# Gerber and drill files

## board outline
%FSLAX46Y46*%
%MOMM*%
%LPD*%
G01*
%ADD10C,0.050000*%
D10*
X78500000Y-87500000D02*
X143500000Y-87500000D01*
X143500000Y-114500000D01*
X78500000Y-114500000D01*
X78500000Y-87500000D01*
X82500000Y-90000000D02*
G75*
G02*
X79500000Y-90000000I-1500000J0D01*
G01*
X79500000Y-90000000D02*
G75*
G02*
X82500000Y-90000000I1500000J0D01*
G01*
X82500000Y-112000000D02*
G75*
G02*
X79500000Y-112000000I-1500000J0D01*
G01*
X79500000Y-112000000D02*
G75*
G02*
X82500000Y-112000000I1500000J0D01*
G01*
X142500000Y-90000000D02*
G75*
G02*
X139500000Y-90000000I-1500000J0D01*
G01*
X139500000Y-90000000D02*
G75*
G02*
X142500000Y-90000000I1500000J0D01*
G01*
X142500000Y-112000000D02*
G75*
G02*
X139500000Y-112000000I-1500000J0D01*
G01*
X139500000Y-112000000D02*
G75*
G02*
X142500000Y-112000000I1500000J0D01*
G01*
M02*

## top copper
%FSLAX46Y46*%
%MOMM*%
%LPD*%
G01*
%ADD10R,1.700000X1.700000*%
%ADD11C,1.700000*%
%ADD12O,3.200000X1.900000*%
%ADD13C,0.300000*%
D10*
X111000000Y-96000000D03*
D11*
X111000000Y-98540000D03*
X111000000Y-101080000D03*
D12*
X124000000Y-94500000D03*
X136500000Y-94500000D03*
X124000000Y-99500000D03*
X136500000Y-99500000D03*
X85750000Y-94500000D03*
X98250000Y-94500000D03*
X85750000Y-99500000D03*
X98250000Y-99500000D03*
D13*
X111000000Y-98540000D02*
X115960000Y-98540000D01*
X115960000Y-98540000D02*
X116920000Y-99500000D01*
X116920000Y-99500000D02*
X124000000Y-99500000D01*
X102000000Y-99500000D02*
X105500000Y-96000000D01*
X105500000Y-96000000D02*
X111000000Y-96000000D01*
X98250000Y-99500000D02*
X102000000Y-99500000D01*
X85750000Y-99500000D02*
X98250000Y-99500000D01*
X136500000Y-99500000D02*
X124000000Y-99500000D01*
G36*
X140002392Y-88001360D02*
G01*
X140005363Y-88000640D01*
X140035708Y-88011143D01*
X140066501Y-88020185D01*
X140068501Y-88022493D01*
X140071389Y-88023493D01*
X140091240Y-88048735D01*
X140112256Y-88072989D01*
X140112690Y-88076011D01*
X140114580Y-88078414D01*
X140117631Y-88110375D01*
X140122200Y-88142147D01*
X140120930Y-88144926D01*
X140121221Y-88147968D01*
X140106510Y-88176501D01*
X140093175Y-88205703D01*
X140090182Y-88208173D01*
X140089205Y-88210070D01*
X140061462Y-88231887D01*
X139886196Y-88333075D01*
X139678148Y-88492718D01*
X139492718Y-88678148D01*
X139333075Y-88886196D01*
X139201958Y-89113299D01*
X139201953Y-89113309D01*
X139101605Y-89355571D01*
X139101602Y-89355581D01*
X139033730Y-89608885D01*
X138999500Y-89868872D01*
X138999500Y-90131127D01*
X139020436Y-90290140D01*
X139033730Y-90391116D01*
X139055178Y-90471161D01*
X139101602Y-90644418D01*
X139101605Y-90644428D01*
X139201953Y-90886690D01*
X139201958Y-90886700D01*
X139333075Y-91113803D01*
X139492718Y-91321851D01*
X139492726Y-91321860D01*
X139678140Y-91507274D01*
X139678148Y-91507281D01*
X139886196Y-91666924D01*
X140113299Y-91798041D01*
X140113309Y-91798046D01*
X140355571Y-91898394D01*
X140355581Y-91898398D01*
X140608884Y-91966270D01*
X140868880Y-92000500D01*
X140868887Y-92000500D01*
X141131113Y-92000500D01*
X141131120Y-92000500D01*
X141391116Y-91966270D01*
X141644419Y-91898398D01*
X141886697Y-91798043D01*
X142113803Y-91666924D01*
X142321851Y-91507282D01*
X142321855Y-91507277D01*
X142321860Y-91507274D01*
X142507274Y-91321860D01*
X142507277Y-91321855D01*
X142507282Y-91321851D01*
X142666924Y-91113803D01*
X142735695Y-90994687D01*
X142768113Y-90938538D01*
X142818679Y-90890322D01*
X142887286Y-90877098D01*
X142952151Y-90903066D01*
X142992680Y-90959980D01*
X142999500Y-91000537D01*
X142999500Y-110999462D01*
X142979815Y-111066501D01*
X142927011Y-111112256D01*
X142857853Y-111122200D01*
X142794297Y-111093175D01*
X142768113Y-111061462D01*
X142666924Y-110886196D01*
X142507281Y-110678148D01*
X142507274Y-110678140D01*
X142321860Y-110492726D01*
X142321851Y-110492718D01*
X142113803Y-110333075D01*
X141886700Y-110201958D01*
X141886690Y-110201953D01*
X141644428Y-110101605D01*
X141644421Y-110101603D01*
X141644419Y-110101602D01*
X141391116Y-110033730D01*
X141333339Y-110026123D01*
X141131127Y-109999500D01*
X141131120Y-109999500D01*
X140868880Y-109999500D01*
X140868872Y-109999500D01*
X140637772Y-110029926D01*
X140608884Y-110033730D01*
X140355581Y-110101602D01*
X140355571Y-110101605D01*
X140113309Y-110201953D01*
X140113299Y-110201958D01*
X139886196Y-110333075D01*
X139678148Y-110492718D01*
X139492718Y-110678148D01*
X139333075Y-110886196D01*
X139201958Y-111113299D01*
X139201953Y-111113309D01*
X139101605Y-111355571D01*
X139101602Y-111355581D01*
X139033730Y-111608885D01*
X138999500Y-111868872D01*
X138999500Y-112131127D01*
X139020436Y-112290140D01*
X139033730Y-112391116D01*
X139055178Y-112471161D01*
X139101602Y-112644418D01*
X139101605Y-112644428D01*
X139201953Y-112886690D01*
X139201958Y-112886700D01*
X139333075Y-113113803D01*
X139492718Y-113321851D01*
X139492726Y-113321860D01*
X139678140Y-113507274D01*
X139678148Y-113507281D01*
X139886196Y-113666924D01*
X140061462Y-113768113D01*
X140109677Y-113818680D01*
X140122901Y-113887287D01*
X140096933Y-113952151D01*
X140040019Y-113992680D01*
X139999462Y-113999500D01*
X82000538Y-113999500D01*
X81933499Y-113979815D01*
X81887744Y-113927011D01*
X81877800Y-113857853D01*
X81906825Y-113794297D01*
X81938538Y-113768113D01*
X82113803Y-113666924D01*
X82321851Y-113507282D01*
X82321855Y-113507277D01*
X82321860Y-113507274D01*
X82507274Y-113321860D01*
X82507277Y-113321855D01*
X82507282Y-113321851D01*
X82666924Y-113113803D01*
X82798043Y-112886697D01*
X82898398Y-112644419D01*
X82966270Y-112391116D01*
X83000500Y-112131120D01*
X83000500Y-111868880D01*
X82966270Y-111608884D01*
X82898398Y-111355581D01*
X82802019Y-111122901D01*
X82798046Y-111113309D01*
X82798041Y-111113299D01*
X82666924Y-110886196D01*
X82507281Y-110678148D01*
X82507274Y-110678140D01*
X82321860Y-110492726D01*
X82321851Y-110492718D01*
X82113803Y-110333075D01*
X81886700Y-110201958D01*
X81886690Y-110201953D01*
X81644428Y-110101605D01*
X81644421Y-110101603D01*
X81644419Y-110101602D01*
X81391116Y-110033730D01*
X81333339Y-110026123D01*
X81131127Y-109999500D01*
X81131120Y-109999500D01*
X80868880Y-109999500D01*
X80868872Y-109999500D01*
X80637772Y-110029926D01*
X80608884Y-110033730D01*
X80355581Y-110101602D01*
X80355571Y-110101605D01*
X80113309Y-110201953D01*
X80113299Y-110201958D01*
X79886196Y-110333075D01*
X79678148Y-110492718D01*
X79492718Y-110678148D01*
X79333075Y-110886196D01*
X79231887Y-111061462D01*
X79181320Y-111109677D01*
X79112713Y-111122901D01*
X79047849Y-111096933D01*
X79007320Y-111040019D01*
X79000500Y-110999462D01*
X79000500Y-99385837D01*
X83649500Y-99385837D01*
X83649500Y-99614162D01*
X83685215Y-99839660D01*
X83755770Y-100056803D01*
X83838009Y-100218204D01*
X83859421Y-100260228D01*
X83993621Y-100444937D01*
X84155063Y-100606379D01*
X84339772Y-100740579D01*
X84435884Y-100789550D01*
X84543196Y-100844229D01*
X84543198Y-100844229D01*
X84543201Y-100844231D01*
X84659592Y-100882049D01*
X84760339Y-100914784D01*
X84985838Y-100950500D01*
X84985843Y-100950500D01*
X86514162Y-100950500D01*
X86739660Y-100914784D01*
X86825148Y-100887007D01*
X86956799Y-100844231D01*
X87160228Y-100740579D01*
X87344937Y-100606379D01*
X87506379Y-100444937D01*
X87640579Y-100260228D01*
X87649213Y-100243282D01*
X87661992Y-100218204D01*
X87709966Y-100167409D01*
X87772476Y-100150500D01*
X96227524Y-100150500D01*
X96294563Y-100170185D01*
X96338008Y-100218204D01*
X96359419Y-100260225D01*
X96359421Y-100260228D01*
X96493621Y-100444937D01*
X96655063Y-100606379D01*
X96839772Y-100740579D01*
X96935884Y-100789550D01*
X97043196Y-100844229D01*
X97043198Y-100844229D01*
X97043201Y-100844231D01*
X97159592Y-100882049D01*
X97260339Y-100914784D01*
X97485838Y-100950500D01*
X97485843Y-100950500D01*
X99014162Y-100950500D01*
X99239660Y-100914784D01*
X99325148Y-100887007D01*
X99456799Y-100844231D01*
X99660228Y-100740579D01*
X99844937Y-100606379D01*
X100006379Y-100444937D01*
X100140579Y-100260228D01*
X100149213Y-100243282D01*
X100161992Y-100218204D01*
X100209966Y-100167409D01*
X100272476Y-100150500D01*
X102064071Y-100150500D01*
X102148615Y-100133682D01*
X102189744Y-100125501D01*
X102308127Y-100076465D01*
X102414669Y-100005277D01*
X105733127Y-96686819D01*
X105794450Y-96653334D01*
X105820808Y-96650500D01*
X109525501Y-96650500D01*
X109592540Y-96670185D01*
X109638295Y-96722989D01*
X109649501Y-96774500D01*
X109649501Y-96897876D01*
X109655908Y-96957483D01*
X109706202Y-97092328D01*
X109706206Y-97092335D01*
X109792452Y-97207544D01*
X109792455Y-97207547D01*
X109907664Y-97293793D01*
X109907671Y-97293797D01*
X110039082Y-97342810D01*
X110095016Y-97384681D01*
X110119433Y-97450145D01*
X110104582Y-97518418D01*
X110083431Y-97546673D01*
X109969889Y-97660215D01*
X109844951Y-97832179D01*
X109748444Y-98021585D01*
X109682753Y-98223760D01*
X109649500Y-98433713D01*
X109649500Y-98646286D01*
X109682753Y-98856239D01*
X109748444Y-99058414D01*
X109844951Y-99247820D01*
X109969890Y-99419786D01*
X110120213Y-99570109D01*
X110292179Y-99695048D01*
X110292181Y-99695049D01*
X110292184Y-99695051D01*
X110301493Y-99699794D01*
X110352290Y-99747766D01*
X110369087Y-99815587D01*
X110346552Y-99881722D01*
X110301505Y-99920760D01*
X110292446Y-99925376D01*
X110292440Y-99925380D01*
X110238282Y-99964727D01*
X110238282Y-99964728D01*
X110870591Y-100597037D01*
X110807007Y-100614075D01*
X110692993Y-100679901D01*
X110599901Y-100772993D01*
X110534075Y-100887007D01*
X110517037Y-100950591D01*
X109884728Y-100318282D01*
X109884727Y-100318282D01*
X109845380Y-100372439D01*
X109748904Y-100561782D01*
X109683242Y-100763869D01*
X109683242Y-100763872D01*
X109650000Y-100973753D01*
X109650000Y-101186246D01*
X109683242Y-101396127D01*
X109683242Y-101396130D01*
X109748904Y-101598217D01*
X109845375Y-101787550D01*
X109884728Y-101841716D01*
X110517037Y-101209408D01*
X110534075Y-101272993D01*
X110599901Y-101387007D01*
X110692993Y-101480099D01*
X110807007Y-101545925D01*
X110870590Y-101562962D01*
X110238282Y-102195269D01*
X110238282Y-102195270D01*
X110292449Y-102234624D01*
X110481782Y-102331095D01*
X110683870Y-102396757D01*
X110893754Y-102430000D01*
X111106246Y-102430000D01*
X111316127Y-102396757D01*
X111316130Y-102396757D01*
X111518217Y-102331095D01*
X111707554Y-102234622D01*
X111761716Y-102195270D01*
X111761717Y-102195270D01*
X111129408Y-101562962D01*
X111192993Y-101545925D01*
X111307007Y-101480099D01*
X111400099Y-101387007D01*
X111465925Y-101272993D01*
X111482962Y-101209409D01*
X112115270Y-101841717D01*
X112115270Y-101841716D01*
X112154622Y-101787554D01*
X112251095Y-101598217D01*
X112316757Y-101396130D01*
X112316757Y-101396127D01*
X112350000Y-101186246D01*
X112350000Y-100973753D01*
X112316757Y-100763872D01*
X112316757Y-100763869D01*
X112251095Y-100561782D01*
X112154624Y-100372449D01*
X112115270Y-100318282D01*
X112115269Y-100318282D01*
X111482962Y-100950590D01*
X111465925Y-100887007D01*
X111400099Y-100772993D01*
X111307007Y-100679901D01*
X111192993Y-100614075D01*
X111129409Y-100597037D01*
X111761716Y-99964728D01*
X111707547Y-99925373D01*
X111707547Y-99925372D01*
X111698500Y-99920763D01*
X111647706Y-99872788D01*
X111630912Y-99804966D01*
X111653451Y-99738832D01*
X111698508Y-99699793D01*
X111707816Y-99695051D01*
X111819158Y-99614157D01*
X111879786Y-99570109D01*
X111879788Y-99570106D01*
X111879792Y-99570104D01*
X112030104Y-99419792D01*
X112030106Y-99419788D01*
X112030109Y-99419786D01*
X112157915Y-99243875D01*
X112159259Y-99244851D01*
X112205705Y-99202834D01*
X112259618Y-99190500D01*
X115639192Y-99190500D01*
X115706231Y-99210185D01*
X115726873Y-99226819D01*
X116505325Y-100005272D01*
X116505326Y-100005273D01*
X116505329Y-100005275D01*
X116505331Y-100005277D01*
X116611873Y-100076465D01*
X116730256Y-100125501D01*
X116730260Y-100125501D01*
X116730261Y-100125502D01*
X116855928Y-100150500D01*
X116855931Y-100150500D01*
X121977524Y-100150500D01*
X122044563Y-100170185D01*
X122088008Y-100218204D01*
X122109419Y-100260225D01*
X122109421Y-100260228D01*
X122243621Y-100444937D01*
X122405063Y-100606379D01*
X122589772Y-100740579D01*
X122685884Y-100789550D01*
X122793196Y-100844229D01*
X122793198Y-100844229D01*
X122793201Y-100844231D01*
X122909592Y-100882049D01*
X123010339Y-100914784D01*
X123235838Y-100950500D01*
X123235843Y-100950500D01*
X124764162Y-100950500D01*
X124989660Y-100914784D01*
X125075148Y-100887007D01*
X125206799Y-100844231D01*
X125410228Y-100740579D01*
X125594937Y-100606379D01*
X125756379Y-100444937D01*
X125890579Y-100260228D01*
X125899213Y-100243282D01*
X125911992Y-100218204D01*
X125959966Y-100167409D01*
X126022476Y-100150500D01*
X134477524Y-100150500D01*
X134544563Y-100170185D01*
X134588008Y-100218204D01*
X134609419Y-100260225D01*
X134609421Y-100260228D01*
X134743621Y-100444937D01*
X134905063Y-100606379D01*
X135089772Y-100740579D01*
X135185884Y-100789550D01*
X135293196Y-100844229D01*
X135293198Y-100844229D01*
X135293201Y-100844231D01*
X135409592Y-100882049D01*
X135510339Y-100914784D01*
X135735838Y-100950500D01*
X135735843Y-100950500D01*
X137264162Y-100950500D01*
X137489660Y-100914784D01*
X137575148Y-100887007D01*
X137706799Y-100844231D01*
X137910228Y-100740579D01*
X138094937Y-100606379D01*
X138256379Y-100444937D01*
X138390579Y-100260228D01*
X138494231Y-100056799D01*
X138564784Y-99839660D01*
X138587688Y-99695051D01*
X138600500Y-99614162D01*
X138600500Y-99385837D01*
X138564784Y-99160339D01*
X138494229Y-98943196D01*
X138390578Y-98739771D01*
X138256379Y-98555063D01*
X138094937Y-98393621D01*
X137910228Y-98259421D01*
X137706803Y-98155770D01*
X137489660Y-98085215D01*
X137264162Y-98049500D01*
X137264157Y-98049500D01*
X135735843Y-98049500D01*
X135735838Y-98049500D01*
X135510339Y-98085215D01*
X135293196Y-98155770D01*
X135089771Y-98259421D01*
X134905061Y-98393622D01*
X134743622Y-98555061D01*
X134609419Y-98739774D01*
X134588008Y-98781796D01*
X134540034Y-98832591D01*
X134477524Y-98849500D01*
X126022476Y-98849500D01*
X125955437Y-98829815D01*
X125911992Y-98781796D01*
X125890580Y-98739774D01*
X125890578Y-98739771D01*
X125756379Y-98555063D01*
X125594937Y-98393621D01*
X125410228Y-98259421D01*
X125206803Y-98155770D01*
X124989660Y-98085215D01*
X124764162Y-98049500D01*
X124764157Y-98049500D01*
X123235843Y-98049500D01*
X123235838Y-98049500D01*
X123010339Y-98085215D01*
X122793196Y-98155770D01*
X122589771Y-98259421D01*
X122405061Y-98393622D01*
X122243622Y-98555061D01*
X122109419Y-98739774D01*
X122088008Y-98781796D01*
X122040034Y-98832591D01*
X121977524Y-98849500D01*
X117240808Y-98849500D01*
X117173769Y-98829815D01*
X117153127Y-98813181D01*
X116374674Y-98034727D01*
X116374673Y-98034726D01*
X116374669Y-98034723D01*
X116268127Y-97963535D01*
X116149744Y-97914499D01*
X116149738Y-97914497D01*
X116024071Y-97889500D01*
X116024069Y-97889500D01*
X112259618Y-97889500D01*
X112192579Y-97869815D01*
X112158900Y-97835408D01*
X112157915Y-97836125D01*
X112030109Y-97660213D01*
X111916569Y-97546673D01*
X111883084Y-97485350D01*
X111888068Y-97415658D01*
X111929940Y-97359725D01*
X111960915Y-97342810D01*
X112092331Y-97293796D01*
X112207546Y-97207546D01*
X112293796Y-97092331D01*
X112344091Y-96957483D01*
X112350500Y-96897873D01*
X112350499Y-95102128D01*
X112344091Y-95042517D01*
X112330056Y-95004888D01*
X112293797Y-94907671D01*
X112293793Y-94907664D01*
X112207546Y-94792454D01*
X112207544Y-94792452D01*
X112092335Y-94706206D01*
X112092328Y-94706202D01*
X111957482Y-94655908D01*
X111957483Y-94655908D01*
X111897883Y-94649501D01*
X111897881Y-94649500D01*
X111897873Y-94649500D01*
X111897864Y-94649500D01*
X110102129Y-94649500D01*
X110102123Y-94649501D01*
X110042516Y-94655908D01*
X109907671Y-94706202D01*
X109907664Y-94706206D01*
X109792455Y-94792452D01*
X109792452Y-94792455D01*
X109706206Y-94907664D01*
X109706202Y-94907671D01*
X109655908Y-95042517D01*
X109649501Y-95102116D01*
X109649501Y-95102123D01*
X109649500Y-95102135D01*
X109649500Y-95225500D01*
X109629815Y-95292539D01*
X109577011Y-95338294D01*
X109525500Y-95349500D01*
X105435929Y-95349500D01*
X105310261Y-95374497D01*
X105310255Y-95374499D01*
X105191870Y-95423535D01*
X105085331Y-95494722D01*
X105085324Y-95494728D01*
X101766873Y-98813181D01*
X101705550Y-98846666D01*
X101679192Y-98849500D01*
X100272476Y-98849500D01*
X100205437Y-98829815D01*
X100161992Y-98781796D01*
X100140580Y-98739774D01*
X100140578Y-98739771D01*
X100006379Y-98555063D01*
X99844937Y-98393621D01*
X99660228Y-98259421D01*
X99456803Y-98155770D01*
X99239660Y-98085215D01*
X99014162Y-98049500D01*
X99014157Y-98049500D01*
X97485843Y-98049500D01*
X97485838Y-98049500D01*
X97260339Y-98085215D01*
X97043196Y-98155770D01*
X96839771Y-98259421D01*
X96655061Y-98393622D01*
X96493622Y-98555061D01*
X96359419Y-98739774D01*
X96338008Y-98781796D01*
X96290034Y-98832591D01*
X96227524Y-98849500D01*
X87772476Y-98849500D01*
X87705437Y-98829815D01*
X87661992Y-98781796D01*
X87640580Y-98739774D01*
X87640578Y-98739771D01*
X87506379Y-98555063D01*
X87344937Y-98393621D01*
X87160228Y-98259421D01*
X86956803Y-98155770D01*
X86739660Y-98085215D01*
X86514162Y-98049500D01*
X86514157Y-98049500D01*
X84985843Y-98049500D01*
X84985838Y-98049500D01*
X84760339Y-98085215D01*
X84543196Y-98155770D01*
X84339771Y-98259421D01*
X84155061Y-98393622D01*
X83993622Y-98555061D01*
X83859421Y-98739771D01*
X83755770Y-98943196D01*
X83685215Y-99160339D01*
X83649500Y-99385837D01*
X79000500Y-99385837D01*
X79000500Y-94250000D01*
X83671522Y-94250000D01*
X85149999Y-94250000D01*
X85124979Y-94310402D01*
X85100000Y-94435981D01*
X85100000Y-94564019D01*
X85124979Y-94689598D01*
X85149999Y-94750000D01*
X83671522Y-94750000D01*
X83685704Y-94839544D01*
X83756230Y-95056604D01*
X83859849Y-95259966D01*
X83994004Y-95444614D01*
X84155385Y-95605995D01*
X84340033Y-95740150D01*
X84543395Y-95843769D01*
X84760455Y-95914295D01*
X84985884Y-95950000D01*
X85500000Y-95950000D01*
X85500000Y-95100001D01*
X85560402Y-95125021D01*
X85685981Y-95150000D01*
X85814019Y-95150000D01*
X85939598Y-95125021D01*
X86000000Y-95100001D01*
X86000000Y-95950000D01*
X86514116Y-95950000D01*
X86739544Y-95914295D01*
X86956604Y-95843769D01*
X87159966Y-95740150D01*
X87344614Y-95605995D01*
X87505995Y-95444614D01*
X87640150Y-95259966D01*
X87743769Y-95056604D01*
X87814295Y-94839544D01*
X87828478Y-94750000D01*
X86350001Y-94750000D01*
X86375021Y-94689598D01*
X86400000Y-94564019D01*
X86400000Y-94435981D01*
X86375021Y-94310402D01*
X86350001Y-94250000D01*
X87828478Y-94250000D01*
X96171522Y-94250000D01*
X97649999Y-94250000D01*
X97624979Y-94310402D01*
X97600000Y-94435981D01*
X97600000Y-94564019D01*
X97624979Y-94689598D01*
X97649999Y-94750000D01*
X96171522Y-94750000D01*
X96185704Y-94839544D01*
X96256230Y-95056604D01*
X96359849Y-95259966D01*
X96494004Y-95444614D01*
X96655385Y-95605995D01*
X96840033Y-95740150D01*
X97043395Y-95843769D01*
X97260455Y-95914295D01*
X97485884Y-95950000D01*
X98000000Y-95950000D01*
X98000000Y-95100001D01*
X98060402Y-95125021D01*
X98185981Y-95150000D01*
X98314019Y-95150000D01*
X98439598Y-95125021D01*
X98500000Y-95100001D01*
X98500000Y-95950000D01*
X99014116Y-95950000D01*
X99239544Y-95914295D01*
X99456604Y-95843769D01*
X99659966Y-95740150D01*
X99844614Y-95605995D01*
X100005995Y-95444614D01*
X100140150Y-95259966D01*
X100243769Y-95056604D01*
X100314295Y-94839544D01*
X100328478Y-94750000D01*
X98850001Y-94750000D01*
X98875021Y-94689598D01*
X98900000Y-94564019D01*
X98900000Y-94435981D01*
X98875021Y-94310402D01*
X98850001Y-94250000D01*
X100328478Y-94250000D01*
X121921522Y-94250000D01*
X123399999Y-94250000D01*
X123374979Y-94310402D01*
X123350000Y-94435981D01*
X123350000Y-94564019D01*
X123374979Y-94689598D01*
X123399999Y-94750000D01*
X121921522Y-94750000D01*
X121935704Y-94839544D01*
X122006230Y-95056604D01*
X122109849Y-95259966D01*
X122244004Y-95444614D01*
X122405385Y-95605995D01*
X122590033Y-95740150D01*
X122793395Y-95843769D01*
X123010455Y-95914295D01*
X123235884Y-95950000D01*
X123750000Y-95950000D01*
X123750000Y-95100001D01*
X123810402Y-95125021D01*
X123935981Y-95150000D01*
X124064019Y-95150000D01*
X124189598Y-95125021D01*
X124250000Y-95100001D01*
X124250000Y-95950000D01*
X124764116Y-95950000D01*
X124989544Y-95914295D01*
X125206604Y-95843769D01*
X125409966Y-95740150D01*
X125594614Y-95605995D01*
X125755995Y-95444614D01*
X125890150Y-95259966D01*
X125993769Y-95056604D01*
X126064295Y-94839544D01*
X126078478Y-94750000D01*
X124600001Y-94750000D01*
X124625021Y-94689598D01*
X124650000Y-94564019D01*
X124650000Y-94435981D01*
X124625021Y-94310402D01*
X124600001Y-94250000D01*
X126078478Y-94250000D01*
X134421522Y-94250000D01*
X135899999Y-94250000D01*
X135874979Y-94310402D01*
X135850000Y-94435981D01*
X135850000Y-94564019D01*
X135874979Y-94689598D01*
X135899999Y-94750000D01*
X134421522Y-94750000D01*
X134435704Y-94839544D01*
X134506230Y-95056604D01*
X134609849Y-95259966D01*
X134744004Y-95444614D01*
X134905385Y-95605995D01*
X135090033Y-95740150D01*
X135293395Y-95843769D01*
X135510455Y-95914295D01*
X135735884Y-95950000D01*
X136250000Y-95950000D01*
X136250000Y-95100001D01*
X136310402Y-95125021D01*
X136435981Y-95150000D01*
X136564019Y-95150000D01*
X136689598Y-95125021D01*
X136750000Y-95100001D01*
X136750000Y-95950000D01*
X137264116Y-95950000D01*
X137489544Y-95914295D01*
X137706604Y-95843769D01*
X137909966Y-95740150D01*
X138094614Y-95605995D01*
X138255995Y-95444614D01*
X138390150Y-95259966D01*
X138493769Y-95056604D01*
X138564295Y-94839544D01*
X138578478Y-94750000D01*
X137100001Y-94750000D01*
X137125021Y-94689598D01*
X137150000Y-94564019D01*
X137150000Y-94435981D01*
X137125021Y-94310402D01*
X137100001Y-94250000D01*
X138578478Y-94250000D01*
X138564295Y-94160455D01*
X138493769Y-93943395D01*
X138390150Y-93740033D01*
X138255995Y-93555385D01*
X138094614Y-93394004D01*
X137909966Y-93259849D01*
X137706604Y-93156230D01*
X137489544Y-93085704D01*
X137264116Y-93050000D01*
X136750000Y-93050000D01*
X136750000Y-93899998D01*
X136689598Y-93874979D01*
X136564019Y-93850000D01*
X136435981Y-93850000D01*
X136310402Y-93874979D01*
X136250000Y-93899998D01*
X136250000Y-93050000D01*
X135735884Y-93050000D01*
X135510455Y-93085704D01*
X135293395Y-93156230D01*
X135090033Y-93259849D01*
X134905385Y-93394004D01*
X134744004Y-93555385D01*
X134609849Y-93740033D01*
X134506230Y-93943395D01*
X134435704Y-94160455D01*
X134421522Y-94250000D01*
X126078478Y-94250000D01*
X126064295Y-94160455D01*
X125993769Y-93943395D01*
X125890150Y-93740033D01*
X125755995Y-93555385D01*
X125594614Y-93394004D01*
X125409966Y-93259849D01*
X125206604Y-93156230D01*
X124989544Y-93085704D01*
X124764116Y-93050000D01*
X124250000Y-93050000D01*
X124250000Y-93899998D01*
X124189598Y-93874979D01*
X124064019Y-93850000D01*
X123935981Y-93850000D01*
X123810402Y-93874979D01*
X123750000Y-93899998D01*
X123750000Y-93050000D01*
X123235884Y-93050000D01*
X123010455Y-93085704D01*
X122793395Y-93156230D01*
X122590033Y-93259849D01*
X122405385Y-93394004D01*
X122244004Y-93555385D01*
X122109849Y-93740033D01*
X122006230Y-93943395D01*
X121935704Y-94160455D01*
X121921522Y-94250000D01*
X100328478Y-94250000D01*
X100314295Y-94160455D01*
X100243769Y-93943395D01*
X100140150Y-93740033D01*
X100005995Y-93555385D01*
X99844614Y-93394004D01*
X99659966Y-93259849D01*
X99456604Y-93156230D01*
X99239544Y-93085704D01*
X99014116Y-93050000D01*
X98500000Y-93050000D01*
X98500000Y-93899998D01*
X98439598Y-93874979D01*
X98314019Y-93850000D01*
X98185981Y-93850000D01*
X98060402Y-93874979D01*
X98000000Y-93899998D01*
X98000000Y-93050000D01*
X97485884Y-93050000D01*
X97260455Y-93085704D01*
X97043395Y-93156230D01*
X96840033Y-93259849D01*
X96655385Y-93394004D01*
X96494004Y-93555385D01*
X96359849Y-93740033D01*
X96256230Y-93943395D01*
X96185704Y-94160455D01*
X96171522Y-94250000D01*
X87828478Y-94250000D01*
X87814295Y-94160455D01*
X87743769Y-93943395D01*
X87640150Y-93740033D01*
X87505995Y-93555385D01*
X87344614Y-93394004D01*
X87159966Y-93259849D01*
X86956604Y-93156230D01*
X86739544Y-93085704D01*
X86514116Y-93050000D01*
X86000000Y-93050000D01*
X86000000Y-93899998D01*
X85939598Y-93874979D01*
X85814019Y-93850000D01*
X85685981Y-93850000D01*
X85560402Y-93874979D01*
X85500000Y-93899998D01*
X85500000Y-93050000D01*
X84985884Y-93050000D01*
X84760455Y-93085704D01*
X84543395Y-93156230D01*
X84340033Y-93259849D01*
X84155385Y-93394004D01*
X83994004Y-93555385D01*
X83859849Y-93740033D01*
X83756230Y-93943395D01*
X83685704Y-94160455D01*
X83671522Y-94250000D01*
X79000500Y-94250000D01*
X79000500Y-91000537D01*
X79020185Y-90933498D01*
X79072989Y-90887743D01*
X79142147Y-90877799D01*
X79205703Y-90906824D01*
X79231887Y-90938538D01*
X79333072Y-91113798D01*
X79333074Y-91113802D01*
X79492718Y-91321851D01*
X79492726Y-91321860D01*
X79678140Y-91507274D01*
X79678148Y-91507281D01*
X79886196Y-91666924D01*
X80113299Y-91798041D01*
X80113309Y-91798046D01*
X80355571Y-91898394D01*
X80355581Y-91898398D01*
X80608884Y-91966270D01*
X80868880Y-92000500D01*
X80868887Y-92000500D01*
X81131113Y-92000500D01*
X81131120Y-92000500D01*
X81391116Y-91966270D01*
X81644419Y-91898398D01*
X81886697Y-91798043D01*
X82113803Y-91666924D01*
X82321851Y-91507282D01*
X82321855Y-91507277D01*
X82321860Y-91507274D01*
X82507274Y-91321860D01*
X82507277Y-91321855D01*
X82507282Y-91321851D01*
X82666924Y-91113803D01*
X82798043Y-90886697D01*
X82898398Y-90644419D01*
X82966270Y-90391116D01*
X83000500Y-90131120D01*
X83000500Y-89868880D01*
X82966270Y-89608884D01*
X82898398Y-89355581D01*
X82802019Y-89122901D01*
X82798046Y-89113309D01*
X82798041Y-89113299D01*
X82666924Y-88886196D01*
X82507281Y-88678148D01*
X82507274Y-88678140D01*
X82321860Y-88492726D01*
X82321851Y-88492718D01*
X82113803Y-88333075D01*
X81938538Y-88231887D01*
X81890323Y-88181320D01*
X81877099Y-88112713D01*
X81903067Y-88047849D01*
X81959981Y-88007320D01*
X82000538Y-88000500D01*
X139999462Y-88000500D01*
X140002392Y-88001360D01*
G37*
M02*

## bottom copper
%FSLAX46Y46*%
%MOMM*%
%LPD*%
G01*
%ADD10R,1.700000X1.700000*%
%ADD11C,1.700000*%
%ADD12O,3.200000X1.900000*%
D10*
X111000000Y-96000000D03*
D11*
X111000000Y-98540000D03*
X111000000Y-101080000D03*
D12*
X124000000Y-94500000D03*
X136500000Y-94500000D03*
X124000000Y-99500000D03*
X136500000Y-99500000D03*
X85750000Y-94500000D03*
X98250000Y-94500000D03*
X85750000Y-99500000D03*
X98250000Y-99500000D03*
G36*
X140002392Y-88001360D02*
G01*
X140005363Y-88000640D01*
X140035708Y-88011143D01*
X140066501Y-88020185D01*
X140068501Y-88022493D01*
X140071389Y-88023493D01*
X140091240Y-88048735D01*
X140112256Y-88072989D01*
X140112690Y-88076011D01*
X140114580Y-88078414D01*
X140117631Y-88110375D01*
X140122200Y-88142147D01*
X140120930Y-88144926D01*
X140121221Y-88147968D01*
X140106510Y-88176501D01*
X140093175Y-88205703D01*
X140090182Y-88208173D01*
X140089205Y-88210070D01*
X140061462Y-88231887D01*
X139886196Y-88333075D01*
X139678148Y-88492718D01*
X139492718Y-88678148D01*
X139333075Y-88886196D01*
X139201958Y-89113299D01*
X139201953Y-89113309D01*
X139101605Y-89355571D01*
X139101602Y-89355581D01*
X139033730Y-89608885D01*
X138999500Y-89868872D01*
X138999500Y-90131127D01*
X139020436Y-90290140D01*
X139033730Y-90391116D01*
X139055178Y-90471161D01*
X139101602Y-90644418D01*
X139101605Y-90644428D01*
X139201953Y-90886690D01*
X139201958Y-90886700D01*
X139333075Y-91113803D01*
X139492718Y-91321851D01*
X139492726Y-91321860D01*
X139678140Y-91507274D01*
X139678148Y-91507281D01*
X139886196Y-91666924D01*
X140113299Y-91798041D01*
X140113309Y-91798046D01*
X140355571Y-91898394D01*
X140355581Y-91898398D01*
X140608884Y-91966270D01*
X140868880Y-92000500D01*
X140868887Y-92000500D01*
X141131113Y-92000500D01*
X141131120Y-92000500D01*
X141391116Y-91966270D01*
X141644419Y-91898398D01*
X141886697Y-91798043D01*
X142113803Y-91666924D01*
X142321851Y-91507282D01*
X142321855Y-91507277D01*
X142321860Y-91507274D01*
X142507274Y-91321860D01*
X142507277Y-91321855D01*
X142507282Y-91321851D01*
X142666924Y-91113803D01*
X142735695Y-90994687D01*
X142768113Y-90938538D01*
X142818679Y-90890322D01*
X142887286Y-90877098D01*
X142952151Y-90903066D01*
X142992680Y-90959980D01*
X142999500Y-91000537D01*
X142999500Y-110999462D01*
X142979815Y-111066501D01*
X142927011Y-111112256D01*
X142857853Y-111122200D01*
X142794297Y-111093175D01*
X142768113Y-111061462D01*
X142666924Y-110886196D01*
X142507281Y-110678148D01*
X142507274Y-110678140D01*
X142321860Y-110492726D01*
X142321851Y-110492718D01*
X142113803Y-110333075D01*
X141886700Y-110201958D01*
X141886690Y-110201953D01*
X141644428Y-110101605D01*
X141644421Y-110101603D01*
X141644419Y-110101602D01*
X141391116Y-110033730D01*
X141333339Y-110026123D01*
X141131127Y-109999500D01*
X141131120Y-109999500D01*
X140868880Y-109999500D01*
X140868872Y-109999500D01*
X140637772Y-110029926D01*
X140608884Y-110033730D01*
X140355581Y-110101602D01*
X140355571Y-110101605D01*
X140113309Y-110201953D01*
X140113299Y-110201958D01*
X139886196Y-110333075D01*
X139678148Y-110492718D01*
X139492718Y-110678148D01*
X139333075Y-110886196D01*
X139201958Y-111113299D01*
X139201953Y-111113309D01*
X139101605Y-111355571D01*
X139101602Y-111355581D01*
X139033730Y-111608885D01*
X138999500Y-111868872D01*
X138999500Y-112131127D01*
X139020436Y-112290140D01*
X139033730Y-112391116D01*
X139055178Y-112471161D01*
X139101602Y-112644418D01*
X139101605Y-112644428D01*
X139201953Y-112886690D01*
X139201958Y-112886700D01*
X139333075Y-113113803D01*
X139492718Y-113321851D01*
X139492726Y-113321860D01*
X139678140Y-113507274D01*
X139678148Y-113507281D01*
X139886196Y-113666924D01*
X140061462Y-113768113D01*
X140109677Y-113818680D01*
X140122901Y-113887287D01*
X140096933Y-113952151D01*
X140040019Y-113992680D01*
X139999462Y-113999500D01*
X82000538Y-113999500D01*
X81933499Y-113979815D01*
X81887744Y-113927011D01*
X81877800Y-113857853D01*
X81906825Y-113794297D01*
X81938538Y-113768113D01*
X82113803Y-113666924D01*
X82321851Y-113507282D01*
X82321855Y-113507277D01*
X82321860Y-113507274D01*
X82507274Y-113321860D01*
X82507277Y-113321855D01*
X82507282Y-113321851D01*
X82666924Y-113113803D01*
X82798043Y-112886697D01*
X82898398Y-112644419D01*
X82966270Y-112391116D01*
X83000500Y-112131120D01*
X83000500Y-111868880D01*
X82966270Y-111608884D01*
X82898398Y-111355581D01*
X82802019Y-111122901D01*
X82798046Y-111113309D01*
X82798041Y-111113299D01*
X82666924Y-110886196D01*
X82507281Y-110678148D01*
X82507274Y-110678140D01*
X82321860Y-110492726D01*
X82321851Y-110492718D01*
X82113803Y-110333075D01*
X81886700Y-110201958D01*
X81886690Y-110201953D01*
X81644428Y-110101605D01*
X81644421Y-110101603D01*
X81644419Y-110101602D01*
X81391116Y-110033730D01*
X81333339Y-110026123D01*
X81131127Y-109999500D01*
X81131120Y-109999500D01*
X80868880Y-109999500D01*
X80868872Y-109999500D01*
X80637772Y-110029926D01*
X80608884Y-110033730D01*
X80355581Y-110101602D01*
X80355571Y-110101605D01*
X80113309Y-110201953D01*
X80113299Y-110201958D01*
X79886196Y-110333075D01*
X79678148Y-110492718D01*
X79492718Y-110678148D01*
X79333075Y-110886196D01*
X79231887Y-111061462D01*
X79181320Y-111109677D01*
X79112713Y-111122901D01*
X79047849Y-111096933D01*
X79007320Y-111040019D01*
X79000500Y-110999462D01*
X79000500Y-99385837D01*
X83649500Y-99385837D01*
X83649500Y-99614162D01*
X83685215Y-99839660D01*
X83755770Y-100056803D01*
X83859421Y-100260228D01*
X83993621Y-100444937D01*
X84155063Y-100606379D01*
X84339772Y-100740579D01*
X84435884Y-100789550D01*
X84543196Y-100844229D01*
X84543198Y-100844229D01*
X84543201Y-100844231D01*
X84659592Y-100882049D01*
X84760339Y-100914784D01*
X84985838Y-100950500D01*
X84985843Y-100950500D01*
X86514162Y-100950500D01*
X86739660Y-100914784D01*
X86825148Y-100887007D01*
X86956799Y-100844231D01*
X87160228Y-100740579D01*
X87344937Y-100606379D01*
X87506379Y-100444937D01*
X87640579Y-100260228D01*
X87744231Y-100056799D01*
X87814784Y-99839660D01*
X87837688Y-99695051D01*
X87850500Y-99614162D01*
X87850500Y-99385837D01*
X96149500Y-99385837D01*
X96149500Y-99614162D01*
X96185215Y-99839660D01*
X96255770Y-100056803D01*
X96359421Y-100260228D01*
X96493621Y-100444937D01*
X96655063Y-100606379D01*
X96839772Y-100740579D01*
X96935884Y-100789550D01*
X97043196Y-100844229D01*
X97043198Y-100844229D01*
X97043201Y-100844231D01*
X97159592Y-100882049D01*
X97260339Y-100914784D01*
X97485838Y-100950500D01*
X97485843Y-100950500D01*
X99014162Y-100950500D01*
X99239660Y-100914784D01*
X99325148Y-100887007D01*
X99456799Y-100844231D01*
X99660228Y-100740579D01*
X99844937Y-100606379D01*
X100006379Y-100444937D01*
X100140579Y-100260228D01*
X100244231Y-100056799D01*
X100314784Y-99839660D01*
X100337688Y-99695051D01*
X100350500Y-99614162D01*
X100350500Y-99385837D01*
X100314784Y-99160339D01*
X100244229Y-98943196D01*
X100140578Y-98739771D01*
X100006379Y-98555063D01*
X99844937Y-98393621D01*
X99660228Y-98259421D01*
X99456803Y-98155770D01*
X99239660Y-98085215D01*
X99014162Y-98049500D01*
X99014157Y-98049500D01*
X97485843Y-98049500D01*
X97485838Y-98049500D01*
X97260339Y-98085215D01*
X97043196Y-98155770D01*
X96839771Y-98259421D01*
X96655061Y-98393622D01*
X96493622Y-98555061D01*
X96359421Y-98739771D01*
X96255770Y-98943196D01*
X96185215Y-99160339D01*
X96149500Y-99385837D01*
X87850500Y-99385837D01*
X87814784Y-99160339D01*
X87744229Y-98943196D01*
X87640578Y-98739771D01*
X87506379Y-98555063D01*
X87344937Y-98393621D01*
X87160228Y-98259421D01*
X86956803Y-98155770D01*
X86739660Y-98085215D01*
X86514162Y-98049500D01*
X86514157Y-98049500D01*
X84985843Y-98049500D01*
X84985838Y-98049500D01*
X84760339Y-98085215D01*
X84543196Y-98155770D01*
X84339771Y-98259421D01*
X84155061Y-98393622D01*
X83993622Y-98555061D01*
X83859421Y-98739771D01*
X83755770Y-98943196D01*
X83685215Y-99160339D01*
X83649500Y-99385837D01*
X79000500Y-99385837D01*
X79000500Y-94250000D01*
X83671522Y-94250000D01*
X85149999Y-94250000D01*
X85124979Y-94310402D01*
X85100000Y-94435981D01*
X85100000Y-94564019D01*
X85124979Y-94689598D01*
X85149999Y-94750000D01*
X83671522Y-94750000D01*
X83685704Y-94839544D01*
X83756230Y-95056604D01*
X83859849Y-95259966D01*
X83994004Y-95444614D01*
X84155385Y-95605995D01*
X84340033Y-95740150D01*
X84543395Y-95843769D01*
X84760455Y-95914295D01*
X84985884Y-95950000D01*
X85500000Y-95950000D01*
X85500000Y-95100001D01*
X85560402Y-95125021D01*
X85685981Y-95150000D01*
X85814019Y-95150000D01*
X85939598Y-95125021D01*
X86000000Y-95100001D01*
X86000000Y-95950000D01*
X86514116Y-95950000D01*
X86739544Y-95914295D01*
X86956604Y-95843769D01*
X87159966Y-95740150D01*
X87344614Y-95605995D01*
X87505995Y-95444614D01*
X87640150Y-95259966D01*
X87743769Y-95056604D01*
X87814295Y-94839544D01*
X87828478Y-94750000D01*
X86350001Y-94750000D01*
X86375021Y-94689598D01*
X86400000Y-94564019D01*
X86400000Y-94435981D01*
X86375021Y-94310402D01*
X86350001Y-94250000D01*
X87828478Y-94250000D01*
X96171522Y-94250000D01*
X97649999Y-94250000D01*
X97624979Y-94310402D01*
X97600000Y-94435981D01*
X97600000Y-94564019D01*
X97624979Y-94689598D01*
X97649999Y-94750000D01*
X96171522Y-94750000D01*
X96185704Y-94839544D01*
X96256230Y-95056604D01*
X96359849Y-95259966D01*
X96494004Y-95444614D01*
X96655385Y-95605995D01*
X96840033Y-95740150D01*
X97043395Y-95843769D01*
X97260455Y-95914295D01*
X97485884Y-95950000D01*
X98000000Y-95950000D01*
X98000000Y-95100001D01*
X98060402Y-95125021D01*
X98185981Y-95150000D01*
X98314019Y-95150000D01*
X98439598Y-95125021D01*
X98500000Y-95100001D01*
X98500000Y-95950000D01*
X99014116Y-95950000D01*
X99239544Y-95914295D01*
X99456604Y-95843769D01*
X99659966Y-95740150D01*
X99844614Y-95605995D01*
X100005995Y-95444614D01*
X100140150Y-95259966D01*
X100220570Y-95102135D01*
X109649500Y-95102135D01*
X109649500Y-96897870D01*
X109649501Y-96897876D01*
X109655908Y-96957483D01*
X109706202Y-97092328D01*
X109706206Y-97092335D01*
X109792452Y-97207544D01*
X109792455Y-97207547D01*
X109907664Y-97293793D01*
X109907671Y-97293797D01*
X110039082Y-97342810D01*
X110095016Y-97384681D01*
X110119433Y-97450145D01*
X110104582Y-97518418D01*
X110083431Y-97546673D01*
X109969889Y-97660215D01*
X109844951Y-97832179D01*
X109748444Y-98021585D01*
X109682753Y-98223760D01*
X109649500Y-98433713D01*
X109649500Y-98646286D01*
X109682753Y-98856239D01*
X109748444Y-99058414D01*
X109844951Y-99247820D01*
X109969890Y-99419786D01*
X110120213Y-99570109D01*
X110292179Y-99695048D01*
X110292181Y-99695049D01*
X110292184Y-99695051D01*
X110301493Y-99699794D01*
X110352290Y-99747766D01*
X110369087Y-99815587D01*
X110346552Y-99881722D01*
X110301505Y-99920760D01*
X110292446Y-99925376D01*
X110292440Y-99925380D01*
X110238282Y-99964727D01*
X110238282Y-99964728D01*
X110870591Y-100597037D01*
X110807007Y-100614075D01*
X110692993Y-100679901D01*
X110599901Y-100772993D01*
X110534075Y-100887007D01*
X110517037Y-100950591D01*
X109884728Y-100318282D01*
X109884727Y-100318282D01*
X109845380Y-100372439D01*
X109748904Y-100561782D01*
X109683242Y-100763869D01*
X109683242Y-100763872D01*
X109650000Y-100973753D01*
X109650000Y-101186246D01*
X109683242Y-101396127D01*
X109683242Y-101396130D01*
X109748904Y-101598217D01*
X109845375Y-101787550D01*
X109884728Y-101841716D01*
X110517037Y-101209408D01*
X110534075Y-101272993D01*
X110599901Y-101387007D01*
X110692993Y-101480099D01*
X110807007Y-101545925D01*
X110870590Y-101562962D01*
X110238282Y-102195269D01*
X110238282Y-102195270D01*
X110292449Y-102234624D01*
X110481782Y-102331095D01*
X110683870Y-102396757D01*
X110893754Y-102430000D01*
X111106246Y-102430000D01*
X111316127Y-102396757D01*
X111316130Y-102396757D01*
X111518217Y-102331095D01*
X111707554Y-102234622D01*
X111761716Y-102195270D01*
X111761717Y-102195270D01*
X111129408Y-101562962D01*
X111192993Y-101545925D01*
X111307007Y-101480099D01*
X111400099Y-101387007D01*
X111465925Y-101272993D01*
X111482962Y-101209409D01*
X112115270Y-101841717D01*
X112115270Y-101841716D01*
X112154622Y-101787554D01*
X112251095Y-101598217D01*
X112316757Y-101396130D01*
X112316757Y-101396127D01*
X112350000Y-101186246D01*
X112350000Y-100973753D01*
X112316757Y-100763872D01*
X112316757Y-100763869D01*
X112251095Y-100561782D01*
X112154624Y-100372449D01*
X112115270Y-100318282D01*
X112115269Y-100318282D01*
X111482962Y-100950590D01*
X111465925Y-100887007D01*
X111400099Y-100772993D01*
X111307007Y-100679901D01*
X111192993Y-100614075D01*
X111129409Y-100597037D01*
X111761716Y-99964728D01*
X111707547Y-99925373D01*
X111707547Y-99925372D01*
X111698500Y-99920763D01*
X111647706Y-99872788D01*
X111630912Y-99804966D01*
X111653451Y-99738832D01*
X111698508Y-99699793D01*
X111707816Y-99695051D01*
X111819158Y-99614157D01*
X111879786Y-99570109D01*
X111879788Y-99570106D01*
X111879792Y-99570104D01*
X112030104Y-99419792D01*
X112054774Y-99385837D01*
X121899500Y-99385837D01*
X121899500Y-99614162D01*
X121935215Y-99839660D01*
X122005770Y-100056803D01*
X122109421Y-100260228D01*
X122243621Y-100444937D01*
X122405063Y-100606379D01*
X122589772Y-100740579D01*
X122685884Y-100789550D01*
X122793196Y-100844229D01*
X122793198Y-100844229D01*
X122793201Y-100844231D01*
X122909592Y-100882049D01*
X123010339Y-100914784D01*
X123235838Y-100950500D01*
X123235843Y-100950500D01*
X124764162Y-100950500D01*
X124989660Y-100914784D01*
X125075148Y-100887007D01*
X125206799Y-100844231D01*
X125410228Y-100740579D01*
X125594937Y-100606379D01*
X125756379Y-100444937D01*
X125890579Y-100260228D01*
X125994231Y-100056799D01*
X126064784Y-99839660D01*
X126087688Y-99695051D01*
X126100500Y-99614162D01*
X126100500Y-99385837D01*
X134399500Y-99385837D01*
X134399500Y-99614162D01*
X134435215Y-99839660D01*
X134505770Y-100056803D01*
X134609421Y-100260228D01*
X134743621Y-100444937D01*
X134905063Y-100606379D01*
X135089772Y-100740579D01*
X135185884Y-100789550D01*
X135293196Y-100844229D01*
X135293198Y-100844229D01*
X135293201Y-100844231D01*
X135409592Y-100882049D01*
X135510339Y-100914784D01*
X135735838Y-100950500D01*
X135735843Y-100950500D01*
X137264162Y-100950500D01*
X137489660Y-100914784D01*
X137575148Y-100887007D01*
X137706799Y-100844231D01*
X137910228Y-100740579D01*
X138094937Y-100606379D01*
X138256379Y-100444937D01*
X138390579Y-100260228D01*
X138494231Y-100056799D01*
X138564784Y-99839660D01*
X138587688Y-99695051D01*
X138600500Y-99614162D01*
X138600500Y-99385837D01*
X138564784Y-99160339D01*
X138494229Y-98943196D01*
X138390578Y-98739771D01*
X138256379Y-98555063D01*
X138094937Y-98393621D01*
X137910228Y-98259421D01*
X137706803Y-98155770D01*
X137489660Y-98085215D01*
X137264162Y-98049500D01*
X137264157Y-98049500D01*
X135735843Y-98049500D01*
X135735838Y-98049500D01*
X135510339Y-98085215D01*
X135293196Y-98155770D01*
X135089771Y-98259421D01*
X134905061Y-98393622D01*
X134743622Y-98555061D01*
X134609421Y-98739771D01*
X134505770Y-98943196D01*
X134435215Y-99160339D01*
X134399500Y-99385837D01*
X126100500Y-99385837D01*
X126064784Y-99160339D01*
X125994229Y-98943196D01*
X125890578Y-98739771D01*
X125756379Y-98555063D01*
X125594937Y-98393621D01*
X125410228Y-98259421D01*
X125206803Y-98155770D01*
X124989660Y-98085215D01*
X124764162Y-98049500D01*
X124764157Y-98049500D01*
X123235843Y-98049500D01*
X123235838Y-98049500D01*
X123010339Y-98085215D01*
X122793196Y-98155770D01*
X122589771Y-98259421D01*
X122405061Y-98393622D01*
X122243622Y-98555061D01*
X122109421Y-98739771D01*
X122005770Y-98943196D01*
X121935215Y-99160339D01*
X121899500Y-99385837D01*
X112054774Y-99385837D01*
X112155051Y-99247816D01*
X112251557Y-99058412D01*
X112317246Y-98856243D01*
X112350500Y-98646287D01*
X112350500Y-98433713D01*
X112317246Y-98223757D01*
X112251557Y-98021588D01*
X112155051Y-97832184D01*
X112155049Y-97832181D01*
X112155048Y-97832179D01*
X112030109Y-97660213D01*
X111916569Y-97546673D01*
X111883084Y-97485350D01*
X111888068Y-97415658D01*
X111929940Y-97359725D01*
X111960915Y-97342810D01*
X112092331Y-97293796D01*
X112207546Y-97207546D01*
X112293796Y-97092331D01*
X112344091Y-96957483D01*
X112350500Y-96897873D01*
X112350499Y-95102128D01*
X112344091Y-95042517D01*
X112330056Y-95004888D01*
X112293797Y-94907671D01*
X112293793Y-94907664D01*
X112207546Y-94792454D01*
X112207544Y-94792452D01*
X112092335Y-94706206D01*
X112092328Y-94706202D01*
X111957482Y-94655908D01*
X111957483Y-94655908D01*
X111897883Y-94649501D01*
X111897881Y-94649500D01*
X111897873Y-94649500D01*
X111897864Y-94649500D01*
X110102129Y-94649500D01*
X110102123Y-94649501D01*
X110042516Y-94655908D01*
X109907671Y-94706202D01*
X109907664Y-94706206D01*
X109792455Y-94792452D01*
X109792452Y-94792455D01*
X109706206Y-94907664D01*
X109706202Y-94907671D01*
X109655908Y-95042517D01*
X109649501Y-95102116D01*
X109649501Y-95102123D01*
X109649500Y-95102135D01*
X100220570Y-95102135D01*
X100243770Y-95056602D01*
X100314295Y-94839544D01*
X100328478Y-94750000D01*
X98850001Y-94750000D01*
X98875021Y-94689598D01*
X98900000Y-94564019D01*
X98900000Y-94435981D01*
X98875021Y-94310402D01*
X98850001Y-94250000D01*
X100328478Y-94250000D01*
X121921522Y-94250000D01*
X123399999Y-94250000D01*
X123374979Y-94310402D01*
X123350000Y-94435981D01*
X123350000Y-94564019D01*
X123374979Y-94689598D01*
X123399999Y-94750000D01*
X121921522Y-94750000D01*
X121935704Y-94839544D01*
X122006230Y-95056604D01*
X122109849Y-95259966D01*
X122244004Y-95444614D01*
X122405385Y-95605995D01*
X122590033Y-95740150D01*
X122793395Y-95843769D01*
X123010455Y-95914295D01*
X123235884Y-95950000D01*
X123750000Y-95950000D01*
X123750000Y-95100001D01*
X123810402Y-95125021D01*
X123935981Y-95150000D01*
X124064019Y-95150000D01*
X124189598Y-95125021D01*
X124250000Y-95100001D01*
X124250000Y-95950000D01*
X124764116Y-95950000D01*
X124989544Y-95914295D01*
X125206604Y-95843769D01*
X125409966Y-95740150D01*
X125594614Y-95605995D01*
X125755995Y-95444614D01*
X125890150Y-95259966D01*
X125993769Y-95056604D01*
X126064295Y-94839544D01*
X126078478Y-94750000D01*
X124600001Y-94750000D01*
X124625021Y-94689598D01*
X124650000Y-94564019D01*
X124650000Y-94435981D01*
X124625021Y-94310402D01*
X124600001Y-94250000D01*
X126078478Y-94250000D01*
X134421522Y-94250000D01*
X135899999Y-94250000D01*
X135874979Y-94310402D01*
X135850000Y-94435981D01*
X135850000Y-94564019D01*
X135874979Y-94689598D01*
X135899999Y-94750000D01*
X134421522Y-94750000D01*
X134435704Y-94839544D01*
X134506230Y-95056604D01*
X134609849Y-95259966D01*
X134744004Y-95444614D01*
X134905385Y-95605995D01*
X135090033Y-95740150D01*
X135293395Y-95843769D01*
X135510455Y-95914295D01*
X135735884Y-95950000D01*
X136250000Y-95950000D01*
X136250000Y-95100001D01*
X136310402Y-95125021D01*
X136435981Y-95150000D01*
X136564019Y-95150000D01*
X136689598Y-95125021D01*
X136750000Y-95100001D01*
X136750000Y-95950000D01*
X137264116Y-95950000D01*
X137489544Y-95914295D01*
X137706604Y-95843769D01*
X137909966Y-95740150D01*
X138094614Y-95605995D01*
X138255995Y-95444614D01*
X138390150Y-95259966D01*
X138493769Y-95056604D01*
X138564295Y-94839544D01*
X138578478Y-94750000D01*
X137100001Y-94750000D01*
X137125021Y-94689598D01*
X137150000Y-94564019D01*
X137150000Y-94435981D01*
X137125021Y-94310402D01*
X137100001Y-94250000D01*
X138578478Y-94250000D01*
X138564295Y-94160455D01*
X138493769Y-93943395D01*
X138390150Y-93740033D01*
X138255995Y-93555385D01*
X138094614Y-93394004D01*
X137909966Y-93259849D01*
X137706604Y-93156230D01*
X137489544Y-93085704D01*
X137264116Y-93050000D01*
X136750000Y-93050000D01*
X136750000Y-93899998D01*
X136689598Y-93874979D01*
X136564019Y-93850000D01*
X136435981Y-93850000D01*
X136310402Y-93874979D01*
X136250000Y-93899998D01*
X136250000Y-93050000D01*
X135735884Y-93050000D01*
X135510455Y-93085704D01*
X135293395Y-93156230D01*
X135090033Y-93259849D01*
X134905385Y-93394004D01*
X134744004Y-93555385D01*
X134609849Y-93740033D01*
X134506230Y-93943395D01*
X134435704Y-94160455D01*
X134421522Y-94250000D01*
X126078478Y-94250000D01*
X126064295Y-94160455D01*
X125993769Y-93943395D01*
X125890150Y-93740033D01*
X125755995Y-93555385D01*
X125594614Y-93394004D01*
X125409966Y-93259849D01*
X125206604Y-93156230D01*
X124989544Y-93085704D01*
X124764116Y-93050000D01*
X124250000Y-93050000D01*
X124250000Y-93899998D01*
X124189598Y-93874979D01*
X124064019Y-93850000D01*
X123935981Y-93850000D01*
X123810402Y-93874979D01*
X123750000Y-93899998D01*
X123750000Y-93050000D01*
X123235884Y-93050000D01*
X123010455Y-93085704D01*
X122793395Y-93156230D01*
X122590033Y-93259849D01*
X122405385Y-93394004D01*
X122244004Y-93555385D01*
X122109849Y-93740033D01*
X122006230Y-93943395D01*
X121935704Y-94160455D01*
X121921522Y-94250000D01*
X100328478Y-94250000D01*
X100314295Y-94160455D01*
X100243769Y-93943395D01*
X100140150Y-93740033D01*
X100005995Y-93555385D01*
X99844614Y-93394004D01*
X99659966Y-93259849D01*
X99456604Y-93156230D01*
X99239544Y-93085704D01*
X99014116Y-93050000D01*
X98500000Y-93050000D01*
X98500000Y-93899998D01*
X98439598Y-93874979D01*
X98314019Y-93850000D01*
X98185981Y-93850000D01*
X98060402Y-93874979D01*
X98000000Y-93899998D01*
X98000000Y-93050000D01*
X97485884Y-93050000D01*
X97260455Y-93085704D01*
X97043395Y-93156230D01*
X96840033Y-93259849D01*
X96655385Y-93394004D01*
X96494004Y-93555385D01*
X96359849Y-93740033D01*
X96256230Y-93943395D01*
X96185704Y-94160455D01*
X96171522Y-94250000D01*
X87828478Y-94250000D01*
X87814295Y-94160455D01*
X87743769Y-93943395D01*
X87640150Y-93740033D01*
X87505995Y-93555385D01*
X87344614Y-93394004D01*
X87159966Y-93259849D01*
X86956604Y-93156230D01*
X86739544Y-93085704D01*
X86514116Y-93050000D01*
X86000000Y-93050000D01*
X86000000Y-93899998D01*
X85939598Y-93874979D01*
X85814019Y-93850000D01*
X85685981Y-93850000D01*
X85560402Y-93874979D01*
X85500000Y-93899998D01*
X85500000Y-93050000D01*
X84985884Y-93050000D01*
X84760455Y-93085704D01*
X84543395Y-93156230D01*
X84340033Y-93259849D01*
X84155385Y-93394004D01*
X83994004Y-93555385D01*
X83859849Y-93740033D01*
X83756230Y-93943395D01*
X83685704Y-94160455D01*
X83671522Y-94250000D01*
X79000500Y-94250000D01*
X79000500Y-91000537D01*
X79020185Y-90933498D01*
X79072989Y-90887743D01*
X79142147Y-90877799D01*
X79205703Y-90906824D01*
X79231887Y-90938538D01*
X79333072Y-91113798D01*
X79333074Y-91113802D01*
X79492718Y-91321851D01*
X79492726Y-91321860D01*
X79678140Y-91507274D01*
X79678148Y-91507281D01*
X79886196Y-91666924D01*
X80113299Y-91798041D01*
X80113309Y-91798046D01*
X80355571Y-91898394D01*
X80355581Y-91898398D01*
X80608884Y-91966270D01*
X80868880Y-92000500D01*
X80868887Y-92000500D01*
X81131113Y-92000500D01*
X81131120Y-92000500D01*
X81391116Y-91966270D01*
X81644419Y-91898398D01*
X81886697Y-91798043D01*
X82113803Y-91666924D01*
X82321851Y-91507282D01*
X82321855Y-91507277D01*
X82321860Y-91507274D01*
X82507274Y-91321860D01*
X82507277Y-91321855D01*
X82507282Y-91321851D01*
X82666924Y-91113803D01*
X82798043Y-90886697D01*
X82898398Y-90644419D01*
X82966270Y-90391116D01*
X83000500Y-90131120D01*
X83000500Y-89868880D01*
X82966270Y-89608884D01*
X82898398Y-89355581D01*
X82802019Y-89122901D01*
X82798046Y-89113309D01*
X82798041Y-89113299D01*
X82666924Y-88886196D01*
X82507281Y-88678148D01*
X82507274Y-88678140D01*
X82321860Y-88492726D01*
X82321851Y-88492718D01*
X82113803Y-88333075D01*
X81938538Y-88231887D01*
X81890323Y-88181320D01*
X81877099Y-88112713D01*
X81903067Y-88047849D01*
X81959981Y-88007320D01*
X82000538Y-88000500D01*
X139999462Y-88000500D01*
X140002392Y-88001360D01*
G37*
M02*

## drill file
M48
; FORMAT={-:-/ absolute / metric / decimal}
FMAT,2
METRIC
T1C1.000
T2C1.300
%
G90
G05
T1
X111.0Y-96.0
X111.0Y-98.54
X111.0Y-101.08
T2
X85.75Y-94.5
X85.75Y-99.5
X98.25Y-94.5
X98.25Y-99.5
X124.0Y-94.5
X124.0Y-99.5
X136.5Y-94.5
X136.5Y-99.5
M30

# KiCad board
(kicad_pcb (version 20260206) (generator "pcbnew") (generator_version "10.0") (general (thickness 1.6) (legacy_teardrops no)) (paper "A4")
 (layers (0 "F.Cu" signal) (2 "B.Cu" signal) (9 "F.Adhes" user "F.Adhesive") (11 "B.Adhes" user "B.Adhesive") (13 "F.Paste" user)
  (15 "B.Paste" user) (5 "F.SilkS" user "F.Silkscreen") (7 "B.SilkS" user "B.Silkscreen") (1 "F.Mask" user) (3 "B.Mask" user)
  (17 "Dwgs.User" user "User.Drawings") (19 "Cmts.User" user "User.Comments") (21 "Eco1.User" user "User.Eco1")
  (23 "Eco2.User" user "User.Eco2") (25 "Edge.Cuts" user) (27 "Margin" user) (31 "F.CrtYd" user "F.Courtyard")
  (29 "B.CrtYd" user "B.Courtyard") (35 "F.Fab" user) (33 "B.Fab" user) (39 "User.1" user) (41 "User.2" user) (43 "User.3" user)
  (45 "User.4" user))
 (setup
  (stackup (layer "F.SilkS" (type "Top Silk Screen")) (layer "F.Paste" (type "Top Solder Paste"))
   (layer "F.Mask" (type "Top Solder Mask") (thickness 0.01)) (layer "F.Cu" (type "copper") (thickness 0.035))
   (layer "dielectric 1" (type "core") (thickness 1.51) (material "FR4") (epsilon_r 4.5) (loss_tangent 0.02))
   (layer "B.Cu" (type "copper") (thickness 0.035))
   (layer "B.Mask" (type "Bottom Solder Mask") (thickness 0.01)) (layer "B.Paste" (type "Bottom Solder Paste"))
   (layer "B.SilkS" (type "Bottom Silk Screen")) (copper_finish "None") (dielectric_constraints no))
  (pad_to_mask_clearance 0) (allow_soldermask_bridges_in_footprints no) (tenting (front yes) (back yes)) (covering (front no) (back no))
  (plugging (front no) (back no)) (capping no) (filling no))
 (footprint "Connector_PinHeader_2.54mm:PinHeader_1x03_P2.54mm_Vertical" (layer "F.Cu") (at 111 96)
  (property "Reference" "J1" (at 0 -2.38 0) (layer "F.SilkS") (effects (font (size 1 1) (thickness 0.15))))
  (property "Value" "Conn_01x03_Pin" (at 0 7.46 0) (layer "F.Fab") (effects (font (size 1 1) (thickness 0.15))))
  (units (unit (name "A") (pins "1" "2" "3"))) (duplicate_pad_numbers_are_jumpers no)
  (pad "1" thru_hole rect (at 0 0) (size 1.7 1.7) (drill 1) (layers "*.Cu" "*.Mask") (remove_unused_layers no) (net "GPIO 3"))
  (pad "2" thru_hole circle (at 0 2.54) (size 1.7 1.7) (drill 1) (layers "*.Cu" "*.Mask") (remove_unused_layers no) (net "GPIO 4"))
  (pad "3" thru_hole circle (at 0 5.08) (size 1.7 1.7) (drill 1) (layers "*.Cu" "*.Mask") (remove_unused_layers no) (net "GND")))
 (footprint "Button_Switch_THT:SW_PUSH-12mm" (layer "F.Cu") (at 124 94.5)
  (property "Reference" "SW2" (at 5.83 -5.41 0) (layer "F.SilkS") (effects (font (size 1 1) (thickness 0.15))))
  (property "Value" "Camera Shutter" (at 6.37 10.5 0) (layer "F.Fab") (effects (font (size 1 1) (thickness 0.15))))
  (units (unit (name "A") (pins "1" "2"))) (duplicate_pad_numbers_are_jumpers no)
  (pad "1" thru_hole oval (at 0 0) (size 3.2 1.9) (drill 1.3) (layers "*.Cu" "*.Mask") (remove_unused_layers no) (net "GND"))
  (pad "1" thru_hole oval (at 12.5 0) (size 3.2 1.9) (drill 1.3) (layers "*.Cu" "*.Mask") (remove_unused_layers no) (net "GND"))
  (pad "2" thru_hole oval (at 0 5) (size 3.2 1.9) (drill 1.3) (layers "*.Cu" "*.Mask") (remove_unused_layers no) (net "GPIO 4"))
  (pad "2" thru_hole oval (at 12.5 5) (size 3.2 1.9) (drill 1.3) (layers "*.Cu" "*.Mask") (remove_unused_layers no) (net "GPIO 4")))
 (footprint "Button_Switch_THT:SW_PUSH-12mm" (layer "F.Cu") (at 85.75 94.5)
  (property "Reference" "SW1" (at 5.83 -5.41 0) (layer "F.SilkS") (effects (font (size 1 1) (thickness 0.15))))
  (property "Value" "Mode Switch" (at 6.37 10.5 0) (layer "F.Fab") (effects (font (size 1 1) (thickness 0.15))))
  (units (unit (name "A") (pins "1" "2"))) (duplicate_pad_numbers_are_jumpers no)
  (pad "1" thru_hole oval (at 0 0) (size 3.2 1.9) (drill 1.3) (layers "*.Cu" "*.Mask") (remove_unused_layers no) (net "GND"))
  (pad "1" thru_hole oval (at 12.5 0) (size 3.2 1.9) (drill 1.3) (layers "*.Cu" "*.Mask") (remove_unused_layers no) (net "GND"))
  (pad "2" thru_hole oval (at 0 5) (size 3.2 1.9) (drill 1.3) (layers "*.Cu" "*.Mask") (remove_unused_layers no) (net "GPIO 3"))
  (pad "2" thru_hole oval (at 12.5 5) (size 3.2 1.9) (drill 1.3) (layers "*.Cu" "*.Mask") (remove_unused_layers no) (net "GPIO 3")))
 (gr_rect (start 78.5 87.5) (end 143.5 114.5) (stroke (width 0.05) (type solid)) (fill no) (layer "Edge.Cuts"))
 (gr_circle (center 81 90) (end 82.5 90) (stroke (width 0.05) (type solid)) (fill no) (layer "Edge.Cuts"))
 (gr_circle (center 81 112) (end 82.5 112) (stroke (width 0.05) (type solid)) (fill no) (layer "Edge.Cuts"))
 (gr_circle (center 141 90) (end 142.5 90) (stroke (width 0.05) (type solid)) (fill no) (layer "Edge.Cuts"))
 (gr_circle (center 141 112) (end 142.5 112) (stroke (width 0.05) (type solid)) (fill no) (layer "Edge.Cuts"))
 (segment (start 105.5 96) (end 111 96) (width 0.3) (layer "F.Cu") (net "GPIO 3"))
 (segment (start 98.25 99.5) (end 102 99.5) (width 0.3) (layer "F.Cu") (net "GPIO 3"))
 (segment (start 102 99.5) (end 105.5 96) (width 0.3) (layer "F.Cu") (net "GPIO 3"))
 (segment (start 85.75 99.5) (end 98.25 99.5) (width 0.3) (layer "F.Cu") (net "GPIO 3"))
 (segment (start 111 98.54) (end 115.96 98.54) (width 0.3) (layer "F.Cu") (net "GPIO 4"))
 (segment (start 116.92 99.5) (end 124 99.5) (width 0.3) (layer "F.Cu") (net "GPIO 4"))
 (segment (start 115.96 98.54) (end 116.92 99.5) (width 0.3) (layer "F.Cu") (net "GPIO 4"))
 (segment (start 136.5 99.5) (end 124 99.5) (width 0.3) (layer "F.Cu") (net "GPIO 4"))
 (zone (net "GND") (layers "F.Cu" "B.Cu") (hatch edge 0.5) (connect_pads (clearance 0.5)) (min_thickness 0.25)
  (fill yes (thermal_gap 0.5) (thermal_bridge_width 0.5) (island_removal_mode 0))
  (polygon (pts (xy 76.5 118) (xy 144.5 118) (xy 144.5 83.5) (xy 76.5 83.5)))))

